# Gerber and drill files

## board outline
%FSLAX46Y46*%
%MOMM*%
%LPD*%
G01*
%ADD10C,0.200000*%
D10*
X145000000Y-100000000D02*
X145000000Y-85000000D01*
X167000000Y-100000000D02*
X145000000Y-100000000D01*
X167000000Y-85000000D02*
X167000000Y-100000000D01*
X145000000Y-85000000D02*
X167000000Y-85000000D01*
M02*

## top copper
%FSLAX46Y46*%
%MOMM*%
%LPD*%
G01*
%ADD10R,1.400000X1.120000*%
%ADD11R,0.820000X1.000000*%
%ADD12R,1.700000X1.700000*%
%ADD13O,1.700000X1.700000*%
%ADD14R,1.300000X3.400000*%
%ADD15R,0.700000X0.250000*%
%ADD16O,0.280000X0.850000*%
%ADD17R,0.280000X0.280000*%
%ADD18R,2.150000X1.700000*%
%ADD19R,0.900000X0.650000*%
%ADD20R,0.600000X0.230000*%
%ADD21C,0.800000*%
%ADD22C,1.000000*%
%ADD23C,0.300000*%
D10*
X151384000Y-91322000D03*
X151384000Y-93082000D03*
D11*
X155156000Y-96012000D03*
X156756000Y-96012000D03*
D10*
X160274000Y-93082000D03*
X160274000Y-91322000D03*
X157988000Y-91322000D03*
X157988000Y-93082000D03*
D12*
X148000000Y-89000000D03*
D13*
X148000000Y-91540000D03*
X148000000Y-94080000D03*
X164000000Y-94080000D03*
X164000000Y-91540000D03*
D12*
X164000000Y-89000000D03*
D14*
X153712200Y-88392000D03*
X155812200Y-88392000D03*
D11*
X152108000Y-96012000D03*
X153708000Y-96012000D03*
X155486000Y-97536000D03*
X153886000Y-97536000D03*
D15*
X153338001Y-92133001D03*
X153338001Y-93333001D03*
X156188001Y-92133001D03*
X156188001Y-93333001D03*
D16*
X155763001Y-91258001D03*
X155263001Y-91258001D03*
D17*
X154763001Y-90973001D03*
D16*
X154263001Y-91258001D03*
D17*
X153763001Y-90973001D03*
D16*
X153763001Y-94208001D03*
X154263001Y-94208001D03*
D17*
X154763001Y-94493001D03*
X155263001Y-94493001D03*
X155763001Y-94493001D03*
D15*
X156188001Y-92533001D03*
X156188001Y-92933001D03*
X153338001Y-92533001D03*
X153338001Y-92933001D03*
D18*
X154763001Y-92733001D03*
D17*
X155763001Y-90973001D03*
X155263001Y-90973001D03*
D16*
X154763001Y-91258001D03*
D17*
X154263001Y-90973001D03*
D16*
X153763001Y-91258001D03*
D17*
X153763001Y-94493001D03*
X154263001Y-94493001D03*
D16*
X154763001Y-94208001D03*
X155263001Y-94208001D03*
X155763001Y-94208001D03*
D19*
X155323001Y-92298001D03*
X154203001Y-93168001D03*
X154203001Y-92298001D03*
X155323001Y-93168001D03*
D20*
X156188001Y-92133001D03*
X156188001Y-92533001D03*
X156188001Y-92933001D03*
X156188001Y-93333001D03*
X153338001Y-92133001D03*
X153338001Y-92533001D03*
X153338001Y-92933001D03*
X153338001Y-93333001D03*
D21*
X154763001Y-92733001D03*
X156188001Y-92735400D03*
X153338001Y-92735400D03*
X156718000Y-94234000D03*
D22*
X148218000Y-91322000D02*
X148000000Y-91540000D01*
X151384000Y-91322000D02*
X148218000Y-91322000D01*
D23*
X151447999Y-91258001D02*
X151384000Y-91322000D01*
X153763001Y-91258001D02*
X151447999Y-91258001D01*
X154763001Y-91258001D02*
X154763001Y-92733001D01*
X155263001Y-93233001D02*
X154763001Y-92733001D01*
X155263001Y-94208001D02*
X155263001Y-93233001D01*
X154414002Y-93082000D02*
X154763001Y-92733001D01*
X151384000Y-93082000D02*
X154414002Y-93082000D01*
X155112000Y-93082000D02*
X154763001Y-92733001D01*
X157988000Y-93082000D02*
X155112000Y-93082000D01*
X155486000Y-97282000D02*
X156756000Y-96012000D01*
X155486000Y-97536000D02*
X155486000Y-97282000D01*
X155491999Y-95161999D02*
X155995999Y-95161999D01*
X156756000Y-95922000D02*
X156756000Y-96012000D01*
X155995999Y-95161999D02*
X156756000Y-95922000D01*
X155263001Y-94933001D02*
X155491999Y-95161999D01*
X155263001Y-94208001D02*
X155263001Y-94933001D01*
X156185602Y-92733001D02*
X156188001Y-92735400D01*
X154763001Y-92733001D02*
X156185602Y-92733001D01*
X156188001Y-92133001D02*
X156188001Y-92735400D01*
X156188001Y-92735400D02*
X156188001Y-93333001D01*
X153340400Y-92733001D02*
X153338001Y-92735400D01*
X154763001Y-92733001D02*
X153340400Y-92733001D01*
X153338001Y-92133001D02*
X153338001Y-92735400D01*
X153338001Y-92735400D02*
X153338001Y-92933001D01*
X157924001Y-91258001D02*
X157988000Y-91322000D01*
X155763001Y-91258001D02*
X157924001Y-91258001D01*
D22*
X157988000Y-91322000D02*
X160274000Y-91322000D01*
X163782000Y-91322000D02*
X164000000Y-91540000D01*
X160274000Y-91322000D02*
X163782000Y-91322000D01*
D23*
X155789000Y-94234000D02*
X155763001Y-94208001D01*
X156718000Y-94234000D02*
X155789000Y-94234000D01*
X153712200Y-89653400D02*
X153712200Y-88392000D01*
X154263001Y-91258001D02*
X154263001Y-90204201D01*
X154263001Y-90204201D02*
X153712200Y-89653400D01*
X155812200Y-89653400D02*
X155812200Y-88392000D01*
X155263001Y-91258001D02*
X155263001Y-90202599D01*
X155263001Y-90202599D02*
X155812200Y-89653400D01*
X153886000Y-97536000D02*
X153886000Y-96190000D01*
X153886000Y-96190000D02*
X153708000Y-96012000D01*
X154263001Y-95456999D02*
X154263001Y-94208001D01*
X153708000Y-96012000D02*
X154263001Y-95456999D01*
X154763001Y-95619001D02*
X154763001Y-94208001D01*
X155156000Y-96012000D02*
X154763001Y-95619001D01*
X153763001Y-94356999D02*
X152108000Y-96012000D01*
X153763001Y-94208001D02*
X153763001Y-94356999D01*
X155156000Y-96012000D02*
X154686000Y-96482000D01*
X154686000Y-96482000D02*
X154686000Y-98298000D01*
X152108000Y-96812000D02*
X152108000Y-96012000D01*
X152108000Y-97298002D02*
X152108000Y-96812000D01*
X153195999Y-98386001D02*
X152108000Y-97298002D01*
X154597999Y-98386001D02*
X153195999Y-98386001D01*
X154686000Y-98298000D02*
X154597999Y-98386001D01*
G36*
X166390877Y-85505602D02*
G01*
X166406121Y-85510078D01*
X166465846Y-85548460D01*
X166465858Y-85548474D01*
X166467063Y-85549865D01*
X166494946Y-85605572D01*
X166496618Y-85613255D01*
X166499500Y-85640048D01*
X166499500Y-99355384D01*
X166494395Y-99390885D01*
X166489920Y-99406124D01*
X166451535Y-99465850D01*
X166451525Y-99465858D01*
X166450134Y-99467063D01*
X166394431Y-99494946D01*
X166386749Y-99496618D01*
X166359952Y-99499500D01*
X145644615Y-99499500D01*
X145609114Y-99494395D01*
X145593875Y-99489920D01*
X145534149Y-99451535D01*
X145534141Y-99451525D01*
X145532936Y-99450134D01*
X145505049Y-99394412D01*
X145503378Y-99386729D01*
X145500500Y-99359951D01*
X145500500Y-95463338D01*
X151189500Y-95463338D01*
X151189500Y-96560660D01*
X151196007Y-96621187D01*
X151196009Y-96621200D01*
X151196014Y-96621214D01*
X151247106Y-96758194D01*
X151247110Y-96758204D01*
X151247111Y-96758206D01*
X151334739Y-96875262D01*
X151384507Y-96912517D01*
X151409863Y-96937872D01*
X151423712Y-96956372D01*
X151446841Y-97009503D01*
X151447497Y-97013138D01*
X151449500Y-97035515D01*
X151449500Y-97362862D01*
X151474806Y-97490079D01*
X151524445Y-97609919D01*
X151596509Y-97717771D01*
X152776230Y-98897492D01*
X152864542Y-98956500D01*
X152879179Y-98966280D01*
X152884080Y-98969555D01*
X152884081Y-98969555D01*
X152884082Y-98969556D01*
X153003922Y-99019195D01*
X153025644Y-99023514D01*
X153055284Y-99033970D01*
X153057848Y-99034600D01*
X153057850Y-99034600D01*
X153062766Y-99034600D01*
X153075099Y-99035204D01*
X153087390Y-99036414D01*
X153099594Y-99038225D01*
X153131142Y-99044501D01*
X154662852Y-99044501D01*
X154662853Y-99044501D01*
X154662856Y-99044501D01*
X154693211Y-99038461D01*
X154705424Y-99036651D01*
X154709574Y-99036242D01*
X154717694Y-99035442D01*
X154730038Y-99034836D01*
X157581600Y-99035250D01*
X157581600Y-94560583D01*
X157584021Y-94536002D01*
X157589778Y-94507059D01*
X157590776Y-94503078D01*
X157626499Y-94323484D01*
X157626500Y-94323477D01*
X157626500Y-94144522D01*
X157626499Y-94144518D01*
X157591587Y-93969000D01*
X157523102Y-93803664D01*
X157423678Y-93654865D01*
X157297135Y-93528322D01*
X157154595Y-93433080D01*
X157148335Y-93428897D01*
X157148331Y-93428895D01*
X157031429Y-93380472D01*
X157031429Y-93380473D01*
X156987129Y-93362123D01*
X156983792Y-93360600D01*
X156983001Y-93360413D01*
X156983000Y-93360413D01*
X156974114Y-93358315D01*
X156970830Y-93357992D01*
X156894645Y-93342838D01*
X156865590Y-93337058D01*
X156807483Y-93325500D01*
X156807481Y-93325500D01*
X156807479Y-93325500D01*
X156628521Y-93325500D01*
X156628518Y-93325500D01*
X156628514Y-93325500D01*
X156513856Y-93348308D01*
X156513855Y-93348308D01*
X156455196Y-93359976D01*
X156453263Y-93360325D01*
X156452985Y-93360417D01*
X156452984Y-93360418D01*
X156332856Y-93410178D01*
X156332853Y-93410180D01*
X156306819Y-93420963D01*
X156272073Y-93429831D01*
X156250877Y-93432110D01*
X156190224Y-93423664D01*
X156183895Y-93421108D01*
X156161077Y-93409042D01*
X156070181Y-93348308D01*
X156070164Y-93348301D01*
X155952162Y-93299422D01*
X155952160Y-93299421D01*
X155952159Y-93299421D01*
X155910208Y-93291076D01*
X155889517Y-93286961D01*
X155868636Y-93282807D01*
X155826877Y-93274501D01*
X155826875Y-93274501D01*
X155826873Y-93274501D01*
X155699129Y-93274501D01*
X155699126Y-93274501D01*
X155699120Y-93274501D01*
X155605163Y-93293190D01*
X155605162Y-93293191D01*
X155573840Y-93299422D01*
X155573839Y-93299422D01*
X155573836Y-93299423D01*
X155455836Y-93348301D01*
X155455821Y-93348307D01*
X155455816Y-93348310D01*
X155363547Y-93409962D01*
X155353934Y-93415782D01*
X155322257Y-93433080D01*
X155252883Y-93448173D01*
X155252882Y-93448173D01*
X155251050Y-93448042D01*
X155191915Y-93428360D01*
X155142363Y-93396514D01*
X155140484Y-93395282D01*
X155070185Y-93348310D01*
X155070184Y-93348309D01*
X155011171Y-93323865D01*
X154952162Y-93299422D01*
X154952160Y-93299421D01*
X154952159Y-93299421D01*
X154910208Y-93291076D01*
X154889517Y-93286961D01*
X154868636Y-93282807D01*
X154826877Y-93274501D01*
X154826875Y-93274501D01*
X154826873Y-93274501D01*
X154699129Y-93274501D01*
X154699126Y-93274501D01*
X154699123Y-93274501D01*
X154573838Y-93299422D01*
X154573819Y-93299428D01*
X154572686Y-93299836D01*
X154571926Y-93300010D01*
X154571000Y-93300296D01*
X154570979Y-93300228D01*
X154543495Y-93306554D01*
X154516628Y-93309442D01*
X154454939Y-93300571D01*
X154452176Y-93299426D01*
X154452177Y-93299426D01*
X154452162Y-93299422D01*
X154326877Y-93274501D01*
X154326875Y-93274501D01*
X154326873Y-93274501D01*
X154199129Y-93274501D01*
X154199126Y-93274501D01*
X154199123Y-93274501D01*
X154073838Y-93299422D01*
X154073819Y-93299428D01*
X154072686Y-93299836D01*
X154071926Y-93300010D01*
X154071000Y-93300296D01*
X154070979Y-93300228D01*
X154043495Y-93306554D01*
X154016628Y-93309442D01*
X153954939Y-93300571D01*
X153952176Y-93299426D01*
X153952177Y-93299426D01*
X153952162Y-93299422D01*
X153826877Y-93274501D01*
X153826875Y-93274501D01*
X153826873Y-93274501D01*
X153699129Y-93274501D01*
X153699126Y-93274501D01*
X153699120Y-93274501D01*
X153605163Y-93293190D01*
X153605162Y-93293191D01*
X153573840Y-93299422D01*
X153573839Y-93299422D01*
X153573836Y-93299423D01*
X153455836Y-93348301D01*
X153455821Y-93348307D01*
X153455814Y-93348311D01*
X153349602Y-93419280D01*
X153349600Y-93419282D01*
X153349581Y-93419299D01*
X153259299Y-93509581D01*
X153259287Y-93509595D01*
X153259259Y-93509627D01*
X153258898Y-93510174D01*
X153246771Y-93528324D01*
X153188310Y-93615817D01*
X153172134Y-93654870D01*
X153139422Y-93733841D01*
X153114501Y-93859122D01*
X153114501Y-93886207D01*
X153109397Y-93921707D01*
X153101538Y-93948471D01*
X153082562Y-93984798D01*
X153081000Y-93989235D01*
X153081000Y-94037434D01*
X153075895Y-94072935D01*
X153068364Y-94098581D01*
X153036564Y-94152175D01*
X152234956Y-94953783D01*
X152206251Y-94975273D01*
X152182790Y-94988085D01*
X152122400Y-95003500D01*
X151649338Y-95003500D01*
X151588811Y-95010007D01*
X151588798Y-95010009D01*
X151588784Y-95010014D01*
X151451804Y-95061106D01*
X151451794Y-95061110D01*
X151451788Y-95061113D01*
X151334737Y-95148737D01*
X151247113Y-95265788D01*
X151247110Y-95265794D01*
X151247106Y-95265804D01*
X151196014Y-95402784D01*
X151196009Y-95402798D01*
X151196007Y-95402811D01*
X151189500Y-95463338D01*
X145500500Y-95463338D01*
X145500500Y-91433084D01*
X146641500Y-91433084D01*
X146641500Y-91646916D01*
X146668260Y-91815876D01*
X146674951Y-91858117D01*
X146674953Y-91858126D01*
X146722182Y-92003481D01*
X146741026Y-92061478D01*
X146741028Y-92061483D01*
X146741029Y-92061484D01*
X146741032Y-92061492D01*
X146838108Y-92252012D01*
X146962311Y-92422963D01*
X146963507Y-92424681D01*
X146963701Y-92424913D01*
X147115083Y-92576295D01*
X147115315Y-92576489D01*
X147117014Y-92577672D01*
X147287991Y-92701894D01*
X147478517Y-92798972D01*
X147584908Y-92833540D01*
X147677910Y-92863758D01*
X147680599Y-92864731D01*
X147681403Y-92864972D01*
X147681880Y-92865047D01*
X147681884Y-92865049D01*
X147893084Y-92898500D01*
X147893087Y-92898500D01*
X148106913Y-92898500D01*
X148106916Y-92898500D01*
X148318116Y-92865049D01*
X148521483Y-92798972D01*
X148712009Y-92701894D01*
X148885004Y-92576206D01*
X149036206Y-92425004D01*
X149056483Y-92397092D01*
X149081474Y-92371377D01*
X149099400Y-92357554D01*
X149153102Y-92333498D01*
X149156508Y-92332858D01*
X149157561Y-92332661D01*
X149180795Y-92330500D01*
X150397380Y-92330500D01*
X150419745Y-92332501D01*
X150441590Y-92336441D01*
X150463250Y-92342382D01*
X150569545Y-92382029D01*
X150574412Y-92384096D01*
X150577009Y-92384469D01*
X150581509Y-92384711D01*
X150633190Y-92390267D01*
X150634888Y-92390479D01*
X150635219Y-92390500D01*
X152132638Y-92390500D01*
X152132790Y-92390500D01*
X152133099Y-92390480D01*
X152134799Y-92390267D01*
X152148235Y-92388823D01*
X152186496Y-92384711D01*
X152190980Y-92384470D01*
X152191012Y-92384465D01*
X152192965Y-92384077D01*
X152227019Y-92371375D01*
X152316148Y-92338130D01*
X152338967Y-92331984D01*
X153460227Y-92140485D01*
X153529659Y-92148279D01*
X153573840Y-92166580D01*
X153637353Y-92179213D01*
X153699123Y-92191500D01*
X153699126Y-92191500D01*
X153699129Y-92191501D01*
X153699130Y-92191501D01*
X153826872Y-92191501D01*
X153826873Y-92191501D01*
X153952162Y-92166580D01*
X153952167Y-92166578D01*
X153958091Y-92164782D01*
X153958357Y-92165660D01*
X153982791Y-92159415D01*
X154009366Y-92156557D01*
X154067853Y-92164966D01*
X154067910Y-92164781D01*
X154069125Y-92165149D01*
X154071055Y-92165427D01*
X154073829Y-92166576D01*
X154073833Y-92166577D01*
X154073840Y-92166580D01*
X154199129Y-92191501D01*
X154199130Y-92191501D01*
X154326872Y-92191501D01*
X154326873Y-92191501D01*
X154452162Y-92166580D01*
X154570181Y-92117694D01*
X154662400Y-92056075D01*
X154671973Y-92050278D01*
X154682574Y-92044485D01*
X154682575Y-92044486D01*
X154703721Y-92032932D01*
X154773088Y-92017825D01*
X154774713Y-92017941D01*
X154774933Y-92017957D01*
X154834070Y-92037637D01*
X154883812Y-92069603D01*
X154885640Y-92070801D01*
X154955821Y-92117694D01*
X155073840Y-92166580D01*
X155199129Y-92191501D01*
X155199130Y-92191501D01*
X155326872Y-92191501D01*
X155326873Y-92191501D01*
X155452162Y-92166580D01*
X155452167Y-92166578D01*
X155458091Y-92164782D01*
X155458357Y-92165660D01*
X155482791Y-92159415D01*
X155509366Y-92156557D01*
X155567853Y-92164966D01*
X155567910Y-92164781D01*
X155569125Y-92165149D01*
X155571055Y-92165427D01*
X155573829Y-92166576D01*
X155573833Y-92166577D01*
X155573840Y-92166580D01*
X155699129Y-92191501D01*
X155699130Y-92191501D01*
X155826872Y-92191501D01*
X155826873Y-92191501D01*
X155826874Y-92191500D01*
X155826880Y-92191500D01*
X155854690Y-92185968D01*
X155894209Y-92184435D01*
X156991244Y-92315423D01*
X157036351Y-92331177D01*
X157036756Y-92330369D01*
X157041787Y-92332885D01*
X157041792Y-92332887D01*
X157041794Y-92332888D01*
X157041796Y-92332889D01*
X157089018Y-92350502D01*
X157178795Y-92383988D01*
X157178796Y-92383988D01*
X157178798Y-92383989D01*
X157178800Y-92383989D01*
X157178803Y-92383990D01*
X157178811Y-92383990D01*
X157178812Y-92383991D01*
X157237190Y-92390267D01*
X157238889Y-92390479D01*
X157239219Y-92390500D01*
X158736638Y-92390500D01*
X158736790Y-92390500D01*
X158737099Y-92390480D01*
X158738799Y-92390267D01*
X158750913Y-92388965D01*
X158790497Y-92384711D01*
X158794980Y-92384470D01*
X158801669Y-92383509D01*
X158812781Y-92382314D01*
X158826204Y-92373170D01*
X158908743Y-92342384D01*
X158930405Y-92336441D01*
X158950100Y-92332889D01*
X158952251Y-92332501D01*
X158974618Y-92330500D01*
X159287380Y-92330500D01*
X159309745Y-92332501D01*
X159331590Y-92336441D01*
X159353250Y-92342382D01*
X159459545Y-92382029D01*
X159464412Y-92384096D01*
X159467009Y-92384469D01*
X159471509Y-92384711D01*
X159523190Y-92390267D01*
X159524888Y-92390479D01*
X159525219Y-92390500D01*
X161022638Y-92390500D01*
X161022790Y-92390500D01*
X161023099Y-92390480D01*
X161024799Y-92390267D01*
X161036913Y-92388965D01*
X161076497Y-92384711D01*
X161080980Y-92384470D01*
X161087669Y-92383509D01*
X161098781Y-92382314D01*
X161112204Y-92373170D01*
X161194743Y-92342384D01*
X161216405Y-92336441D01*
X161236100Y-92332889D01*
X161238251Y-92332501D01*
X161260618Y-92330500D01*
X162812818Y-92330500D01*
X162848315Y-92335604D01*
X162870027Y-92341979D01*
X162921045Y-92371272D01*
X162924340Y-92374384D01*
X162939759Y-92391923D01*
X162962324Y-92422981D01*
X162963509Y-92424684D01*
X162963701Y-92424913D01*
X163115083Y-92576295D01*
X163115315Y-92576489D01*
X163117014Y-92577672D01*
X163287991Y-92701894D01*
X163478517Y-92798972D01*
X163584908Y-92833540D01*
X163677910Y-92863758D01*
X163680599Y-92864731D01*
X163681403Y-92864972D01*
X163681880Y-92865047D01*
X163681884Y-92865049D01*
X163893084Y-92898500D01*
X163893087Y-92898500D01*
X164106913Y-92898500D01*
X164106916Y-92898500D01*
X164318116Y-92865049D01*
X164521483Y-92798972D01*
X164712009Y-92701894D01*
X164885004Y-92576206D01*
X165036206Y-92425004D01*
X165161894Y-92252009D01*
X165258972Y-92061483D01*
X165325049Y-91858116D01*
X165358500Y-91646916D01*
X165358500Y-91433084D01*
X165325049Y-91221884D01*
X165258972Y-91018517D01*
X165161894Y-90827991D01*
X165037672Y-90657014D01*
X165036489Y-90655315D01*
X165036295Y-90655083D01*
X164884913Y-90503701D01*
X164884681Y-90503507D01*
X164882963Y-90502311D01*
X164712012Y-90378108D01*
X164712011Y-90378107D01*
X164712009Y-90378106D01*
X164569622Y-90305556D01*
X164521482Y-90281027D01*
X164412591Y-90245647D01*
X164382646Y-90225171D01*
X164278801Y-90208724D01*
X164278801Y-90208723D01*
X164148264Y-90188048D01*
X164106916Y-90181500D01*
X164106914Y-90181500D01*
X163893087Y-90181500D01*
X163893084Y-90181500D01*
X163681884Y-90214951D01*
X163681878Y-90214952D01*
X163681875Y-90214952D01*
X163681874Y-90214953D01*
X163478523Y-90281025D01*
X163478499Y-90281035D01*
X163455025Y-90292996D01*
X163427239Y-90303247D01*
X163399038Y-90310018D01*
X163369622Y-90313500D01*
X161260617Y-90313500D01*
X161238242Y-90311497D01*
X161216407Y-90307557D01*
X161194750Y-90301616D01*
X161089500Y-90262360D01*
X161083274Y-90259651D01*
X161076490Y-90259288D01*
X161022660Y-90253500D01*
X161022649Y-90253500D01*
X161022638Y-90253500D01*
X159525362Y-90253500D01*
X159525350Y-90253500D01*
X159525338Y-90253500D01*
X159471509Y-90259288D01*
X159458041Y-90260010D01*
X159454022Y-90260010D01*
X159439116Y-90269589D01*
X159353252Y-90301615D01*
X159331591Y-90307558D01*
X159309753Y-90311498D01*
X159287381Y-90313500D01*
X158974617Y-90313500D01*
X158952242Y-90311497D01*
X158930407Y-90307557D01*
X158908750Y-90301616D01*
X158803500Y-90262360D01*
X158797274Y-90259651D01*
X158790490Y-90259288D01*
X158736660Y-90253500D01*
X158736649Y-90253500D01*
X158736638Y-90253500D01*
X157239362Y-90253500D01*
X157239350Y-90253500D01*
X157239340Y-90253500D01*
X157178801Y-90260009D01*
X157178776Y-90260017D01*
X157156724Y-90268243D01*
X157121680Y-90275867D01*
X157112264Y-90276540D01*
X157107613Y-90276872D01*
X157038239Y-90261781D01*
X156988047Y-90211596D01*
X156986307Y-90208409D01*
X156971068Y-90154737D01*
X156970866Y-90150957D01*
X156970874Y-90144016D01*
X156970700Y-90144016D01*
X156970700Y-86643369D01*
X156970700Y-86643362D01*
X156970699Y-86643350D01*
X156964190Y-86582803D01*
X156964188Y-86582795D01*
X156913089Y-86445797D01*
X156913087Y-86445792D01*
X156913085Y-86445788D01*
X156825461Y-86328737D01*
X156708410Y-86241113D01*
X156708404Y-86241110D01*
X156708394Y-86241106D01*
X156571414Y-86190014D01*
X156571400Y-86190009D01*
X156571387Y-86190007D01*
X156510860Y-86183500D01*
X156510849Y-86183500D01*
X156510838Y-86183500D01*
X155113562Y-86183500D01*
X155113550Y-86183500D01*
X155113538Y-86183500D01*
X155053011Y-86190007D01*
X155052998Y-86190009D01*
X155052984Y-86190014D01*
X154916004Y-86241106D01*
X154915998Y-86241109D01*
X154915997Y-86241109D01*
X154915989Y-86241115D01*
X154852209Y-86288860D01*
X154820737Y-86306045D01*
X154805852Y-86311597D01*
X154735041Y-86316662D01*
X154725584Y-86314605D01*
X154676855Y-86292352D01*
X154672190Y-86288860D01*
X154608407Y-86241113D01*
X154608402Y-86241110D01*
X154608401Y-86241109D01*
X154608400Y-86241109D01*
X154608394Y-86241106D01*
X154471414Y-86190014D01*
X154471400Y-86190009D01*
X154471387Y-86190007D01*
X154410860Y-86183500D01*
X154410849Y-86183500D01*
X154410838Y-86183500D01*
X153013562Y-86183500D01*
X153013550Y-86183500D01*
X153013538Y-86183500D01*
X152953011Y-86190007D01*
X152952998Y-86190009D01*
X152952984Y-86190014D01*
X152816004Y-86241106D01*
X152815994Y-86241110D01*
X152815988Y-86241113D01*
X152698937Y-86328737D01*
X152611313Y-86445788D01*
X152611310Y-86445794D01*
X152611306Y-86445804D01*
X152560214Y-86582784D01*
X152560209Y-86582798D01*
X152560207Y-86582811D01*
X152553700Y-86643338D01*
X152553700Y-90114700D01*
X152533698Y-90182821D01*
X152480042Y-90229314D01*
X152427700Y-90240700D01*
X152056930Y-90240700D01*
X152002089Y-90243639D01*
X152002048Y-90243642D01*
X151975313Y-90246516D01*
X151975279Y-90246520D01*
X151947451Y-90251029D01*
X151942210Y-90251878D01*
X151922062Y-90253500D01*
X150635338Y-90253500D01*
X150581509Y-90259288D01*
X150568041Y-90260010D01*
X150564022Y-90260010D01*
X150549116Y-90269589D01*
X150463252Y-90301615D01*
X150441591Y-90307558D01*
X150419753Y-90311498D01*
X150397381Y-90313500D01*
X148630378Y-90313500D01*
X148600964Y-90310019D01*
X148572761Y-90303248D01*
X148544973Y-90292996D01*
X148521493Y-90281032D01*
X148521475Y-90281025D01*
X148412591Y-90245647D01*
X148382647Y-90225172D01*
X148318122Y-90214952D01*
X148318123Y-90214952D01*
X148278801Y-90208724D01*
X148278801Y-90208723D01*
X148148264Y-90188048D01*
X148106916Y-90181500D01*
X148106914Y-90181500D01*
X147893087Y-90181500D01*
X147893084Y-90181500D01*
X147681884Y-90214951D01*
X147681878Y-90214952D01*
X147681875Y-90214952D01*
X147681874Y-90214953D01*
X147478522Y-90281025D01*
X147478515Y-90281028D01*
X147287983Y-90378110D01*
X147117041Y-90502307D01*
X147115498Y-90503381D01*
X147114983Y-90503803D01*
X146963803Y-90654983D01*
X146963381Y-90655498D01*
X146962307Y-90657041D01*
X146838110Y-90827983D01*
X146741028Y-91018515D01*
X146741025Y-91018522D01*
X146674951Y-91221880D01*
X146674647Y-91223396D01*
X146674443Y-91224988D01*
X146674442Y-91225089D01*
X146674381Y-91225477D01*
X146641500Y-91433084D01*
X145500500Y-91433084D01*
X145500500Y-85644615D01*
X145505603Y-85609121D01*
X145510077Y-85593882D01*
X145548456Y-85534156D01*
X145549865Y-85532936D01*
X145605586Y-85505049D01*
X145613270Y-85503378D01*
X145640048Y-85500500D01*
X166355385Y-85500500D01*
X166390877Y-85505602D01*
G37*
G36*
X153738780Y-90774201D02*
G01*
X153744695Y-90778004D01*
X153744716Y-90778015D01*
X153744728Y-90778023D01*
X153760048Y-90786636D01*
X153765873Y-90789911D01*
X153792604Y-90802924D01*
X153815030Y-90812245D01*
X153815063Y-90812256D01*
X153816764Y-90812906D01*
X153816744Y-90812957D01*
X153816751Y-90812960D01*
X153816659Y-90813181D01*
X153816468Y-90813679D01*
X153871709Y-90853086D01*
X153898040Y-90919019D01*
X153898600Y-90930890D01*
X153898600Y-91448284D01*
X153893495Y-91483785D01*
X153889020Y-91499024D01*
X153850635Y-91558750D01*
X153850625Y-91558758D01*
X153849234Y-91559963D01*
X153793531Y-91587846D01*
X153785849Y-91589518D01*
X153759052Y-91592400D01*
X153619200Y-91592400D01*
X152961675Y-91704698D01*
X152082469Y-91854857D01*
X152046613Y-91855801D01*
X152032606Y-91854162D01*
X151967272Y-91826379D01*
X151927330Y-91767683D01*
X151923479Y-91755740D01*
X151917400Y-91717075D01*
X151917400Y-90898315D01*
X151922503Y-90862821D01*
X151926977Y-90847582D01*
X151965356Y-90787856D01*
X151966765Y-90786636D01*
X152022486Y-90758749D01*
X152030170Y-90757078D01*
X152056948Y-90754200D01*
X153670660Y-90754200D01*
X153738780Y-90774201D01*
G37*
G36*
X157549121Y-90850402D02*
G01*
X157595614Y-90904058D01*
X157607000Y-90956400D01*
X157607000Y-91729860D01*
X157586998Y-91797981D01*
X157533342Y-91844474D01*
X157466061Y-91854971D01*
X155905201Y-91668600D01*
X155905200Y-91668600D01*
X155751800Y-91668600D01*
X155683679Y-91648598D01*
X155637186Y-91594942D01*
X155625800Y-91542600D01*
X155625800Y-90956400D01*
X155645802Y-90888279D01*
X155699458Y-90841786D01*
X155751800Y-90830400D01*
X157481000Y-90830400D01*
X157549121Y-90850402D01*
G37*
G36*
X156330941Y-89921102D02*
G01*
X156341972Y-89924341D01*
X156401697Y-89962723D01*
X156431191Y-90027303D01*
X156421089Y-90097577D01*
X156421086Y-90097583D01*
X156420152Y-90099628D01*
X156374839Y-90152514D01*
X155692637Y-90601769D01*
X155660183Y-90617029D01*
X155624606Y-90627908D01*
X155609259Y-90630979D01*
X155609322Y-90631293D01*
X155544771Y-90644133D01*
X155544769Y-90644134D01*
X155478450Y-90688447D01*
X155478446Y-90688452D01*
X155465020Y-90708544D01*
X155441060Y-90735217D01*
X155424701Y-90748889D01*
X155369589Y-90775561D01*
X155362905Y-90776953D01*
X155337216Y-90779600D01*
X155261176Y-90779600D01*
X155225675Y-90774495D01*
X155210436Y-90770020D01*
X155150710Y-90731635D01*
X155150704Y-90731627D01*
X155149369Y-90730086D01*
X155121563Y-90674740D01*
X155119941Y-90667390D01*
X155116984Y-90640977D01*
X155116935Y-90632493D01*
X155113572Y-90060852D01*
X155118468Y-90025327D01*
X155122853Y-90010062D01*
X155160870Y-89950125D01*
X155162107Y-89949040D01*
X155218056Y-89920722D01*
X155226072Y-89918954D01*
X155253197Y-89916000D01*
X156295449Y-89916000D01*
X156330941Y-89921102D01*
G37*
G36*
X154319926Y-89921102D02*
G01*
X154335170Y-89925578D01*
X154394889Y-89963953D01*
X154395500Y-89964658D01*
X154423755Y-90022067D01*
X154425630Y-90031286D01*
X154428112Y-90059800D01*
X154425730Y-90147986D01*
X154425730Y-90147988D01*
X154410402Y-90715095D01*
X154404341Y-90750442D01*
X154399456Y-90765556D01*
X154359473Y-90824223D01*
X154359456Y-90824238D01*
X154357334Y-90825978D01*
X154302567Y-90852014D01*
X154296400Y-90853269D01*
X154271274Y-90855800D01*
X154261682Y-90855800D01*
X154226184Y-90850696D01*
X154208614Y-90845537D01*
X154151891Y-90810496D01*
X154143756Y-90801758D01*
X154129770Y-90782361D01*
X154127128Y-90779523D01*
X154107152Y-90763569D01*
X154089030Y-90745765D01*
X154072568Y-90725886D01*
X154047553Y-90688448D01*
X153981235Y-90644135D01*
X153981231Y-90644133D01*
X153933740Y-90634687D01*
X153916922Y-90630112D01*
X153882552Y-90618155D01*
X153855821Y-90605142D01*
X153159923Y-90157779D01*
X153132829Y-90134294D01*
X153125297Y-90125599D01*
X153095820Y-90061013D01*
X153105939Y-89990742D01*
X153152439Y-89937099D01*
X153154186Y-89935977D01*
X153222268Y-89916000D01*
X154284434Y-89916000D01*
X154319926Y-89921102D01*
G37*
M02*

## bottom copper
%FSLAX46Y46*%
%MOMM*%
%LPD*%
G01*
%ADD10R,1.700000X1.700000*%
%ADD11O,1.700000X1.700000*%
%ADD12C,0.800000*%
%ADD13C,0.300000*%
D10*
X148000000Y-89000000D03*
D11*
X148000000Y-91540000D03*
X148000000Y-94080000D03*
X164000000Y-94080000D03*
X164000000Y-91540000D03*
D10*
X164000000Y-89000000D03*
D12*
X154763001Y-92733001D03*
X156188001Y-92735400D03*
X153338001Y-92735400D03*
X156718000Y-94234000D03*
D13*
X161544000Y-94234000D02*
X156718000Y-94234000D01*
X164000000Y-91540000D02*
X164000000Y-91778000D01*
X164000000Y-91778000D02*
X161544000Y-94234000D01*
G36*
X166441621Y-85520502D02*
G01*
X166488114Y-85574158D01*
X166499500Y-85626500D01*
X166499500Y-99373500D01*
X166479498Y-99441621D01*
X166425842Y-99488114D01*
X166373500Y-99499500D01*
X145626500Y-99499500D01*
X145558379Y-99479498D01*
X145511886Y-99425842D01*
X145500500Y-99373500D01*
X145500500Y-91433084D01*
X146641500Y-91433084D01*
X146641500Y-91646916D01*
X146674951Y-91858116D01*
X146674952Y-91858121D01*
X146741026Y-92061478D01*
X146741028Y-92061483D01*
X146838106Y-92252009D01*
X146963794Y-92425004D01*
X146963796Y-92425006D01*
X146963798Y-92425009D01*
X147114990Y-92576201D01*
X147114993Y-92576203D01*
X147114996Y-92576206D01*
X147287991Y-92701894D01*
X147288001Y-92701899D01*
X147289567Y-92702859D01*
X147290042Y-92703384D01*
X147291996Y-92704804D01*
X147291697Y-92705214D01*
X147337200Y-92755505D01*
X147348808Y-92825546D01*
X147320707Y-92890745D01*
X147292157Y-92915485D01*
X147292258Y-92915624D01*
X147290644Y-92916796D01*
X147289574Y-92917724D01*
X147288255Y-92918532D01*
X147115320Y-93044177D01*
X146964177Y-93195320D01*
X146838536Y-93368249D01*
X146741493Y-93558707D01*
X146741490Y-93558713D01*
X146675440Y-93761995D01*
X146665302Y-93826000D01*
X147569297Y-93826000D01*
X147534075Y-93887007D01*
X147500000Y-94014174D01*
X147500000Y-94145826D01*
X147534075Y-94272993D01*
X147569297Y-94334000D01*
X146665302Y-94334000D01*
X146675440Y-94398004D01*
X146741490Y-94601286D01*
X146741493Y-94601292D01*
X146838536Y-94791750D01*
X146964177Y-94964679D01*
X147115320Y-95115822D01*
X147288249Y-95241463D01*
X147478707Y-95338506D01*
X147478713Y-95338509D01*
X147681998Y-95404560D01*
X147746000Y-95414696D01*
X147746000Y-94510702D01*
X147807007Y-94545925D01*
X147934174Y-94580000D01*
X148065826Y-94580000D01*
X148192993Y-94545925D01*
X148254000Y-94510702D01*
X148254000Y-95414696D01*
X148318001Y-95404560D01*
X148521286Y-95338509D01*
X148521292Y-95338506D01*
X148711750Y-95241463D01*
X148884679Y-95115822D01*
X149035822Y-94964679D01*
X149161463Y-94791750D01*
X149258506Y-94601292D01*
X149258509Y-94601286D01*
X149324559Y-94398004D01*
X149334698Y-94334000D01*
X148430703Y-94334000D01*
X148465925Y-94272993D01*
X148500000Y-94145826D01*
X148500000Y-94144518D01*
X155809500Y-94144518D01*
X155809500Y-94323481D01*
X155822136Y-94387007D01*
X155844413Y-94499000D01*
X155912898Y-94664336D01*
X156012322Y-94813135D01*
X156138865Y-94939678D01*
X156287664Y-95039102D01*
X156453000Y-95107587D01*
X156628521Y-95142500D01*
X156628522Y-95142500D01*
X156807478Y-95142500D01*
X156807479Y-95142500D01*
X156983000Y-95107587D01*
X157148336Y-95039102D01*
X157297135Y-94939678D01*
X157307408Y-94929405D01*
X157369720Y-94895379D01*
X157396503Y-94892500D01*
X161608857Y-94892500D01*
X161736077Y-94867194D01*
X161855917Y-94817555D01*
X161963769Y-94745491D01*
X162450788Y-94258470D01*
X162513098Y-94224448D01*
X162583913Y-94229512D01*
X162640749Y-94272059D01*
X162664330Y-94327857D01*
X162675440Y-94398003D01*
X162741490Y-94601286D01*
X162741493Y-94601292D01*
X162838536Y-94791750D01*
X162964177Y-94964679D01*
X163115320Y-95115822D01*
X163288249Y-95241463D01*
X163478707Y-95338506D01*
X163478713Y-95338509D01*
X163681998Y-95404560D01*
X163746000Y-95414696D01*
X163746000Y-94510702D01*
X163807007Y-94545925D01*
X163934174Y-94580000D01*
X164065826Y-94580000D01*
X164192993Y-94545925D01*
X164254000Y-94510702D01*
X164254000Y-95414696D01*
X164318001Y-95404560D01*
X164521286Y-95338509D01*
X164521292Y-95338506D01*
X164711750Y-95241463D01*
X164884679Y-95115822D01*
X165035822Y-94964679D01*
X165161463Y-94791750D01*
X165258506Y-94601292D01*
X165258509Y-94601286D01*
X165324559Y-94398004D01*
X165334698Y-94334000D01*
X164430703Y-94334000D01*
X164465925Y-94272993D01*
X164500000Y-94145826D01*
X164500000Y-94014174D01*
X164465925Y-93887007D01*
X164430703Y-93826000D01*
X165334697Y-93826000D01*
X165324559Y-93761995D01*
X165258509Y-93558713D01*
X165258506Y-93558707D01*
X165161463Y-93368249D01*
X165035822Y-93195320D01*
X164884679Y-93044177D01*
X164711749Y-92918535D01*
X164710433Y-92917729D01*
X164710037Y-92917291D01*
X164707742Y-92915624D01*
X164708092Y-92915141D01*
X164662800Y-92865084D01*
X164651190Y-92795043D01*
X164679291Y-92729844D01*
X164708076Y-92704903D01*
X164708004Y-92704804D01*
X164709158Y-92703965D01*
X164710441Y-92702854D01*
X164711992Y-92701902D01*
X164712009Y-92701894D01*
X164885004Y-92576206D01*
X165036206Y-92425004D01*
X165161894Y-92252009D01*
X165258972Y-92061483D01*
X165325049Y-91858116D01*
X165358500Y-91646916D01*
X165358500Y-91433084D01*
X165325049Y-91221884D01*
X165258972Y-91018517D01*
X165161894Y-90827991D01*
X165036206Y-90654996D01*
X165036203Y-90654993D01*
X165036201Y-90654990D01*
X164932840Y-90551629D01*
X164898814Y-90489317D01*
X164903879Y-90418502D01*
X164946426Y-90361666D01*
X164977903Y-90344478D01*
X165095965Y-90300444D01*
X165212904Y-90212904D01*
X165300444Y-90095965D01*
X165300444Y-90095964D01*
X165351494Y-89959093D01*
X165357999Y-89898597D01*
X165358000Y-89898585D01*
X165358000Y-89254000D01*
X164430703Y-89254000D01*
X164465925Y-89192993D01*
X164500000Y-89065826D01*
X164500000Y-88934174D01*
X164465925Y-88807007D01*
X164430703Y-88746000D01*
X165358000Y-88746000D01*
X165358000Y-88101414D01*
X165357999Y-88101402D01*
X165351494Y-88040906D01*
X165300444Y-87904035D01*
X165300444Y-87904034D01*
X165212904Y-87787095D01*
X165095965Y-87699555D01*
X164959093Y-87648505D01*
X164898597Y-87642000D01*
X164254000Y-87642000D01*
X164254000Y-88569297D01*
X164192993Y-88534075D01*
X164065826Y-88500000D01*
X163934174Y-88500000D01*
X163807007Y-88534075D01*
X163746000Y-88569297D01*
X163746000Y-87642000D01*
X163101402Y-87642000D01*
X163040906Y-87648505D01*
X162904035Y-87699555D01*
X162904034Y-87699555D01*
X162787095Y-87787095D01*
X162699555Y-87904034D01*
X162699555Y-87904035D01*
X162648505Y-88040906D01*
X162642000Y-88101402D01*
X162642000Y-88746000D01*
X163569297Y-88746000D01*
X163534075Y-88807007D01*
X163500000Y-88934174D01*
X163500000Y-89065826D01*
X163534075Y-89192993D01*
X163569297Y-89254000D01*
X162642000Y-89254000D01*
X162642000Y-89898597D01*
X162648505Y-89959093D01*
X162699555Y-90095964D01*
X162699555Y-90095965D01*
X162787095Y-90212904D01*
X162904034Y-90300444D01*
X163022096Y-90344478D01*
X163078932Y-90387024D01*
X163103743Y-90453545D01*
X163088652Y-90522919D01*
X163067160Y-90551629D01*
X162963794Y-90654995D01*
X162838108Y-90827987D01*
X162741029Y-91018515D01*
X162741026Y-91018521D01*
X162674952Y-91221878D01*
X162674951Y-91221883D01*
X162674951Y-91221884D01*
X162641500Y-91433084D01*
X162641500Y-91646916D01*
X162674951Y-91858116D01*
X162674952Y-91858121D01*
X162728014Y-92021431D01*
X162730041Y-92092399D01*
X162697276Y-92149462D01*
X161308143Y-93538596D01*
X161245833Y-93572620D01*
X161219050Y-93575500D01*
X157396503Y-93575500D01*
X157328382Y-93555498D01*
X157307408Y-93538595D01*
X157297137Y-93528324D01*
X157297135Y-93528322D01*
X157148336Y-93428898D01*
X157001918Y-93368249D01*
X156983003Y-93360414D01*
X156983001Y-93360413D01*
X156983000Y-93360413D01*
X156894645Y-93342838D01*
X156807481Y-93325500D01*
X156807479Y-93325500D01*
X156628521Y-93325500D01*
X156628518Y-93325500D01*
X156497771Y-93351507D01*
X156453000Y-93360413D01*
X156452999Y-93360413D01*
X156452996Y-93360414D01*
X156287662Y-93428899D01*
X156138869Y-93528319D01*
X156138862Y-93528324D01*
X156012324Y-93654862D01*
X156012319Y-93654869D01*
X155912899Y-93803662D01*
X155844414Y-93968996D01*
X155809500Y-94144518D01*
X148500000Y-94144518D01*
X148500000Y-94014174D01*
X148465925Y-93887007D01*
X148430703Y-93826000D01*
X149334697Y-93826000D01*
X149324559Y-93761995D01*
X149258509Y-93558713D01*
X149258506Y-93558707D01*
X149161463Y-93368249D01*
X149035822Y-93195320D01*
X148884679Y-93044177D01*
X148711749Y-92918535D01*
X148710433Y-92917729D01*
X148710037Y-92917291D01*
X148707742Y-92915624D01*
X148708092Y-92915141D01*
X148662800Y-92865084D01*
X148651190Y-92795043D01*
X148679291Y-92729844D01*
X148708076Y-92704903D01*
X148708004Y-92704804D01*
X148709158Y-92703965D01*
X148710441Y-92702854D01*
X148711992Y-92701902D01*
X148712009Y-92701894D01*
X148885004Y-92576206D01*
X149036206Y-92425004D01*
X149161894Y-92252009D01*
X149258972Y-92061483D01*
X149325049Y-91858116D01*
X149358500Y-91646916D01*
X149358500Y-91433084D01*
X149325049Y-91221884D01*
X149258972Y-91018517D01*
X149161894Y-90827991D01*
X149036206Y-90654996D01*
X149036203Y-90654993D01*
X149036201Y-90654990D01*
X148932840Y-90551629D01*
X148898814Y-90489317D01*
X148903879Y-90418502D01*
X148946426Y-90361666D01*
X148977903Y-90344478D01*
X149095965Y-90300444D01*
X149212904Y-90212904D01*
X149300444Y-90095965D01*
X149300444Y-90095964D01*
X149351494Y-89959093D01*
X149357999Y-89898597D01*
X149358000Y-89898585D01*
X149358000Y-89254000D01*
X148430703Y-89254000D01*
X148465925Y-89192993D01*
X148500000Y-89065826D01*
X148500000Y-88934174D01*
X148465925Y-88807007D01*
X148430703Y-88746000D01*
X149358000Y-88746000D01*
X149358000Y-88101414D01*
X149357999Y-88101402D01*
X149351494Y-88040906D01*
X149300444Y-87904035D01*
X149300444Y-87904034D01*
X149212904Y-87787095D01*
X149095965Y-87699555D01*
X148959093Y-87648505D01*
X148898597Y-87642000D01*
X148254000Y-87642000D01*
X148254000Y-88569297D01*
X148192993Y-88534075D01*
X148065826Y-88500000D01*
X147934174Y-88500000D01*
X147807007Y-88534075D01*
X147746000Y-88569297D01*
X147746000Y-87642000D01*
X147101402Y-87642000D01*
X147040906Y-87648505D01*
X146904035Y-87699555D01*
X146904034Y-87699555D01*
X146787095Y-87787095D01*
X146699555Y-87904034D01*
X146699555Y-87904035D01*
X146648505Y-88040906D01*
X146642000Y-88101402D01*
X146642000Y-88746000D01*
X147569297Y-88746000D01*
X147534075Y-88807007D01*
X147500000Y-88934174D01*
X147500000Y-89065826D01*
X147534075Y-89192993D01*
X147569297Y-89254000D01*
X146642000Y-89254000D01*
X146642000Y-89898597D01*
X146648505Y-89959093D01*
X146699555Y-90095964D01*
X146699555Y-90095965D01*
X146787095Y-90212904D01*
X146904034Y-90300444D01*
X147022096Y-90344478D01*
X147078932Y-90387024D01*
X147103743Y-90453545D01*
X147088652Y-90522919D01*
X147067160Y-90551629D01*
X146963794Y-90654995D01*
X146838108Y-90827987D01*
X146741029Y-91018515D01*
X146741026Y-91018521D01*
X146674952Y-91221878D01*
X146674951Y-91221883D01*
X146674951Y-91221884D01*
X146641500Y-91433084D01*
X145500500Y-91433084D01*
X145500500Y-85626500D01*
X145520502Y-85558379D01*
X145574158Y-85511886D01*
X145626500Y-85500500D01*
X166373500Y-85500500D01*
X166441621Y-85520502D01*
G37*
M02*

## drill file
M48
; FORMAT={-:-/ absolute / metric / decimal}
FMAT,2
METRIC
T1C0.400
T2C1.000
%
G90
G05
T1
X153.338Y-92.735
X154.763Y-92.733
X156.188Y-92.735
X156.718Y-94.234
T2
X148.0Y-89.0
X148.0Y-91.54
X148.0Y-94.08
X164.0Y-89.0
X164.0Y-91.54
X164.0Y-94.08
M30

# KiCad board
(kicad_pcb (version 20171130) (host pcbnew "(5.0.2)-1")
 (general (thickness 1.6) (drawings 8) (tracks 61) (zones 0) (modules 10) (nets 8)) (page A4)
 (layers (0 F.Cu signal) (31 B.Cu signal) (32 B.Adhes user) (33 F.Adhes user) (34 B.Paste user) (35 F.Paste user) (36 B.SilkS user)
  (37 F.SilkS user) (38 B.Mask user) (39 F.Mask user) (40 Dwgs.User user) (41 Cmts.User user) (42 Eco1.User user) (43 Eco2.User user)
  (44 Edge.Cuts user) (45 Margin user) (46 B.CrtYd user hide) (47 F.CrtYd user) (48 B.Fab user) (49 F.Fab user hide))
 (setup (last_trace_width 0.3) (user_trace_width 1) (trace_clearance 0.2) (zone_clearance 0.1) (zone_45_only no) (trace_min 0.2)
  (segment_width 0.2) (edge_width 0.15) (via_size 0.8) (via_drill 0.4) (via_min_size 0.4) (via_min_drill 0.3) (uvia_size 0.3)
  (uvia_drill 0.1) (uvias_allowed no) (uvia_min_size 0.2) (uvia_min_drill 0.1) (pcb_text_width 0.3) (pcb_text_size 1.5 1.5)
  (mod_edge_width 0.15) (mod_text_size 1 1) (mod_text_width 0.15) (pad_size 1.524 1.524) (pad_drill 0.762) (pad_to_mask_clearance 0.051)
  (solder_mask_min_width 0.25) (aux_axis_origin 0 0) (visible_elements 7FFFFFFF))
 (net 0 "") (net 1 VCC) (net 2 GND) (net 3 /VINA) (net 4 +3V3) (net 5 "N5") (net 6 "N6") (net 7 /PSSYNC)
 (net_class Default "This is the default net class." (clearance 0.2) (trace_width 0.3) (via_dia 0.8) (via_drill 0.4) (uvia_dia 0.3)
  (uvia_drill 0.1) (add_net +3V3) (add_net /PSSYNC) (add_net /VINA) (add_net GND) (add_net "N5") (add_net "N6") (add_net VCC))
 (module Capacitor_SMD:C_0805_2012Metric (layer F.Cu) (at 151.384 92.202 270)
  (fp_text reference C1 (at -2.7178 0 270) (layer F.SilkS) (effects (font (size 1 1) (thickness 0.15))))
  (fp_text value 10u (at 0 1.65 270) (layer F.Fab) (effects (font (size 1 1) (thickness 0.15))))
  (pad 1 smd rect (at -0.88 0 270) (size 1.12 1.4) (layers F.Cu F.Paste F.Mask) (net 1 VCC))
  (pad 2 smd rect (at 0.88 0 270) (size 1.12 1.4) (layers F.Cu F.Paste F.Mask) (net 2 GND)))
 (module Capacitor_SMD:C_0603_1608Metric (layer F.Cu) (at 155.956 96.012)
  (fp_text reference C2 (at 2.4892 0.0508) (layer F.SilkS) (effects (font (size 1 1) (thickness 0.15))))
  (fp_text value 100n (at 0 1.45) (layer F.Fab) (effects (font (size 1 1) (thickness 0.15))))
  (pad 1 smd rect (at -0.8 0) (size 0.82 1) (layers F.Cu F.Paste F.Mask) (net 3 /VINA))
  (pad 2 smd rect (at 0.8 0) (size 0.82 1) (layers F.Cu F.Paste F.Mask) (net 2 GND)))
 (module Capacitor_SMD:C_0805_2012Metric (layer F.Cu) (at 160.274 92.202 270)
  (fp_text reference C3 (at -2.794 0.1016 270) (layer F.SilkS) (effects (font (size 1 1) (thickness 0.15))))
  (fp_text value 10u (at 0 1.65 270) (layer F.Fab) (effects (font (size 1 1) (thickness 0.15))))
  (pad 2 smd rect (at 0.88 0 270) (size 1.12 1.4) (layers F.Cu F.Paste F.Mask) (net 2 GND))
  (pad 1 smd rect (at -0.88 0 270) (size 1.12 1.4) (layers F.Cu F.Paste F.Mask) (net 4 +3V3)))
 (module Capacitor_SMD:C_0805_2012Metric (layer F.Cu) (at 157.988 92.202 270)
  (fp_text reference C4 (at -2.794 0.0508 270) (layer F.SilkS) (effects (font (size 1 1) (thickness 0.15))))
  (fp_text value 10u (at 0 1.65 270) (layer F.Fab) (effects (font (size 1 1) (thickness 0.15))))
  (pad 1 smd rect (at -0.88 0 270) (size 1.12 1.4) (layers F.Cu F.Paste F.Mask) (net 4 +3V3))
  (pad 2 smd rect (at 0.88 0 270) (size 1.12 1.4) (layers F.Cu F.Paste F.Mask) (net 2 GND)))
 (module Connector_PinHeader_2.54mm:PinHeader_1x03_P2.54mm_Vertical (layer F.Cu) (at 148 89)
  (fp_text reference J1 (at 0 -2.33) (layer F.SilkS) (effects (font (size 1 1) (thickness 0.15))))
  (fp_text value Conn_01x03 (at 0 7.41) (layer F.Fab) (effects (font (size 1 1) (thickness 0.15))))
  (pad 1 thru_hole rect (at 0 0) (size 1.7 1.7) (drill 1) (layers *.Cu *.Mask) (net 2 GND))
  (pad 2 thru_hole oval (at 0 2.54) (size 1.7 1.7) (drill 1) (layers *.Cu *.Mask) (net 1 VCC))
  (pad 3 thru_hole oval (at 0 5.08) (size 1.7 1.7) (drill 1) (layers *.Cu *.Mask) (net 2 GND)))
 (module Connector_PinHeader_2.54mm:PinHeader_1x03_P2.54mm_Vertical (layer F.Cu) (at 164 89)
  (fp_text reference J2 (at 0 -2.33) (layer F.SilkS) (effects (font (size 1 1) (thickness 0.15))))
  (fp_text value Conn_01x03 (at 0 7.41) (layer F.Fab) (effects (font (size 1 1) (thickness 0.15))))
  (pad 3 thru_hole oval (at 0 5.08) (size 1.7 1.7) (drill 1) (layers *.Cu *.Mask) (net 2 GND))
  (pad 2 thru_hole oval (at 0 2.54) (size 1.7 1.7) (drill 1) (layers *.Cu *.Mask) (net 4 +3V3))
  (pad 1 thru_hole rect (at 0 0) (size 1.7 1.7) (drill 1) (layers *.Cu *.Mask) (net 2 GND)))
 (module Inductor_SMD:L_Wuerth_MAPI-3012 (layer F.Cu) (at 154.7622 88.392)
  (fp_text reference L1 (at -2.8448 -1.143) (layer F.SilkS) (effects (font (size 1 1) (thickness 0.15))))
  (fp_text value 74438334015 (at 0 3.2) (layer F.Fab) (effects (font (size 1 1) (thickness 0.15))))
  (pad 1 smd rect (at -1.05 0) (size 1.3 3.4) (layers F.Cu F.Paste F.Mask) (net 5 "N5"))
  (pad 2 smd rect (at 1.05 0) (size 1.3 3.4) (layers F.Cu F.Paste F.Mask) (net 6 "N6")))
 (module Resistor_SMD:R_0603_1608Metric (layer F.Cu) (at 152.908 96.012)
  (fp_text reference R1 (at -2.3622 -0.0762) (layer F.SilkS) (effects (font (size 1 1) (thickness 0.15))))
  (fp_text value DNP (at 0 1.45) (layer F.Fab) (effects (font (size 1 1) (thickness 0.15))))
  (pad 1 smd rect (at -0.8 0) (size 0.82 1) (layers F.Cu F.Paste F.Mask) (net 3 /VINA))
  (pad 2 smd rect (at 0.8 0) (size 0.82 1) (layers F.Cu F.Paste F.Mask) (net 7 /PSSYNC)))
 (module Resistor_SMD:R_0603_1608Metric (layer F.Cu) (at 154.686 97.536)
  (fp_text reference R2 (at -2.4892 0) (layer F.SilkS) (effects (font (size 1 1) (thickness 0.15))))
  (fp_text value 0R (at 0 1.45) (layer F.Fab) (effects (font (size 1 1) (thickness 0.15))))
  (pad 2 smd rect (at 0.8 0) (size 0.82 1) (layers F.Cu F.Paste F.Mask) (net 2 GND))
  (pad 1 smd rect (at -0.8 0) (size 0.82 1) (layers F.Cu F.Paste F.Mask) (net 7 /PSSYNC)))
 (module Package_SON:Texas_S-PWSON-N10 (layer F.Cu) (at 154.763001 92.733001 270)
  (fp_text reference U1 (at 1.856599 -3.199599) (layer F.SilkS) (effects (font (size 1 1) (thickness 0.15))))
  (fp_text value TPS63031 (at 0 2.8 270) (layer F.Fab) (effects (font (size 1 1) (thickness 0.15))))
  (pad 11 smd rect (at -0.6 1.425 270) (size 0.25 0.7) (layers F.Cu F.Mask) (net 2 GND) (solder_paste_margin -0.05))
  (pad 11 smd rect (at 0.6 1.425 270) (size 0.25 0.7) (layers F.Cu F.Mask) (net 2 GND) (solder_paste_margin -0.05))
  (pad 11 smd rect (at -0.6 -1.425 270) (size 0.25 0.7) (layers F.Cu F.Mask) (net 2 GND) (solder_paste_margin -0.05))
  (pad 11 smd rect (at 0.6 -1.425 270) (size 0.25 0.7) (layers F.Cu F.Mask) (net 2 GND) (solder_paste_margin -0.05))
  (pad 1 smd oval (at -1.475 -1 270) (size 0.85 0.28) (layers F.Cu F.Paste F.Mask) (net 4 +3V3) (solder_mask_margin 0.07)
   (solder_paste_margin -0.025))
  (pad 2 smd oval (at -1.475 -0.5 270) (size 0.85 0.28) (layers F.Cu F.Paste F.Mask) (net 6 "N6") (solder_mask_margin 0.07)
   (solder_paste_margin -0.025))
  (pad 3 smd rect (at -1.76 0 270) (size 0.28 0.28) (layers F.Cu F.Paste F.Mask) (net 2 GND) (solder_mask_margin 0.07)
   (solder_paste_margin -0.025))
  (pad 4 smd oval (at -1.475 0.5 270) (size 0.85 0.28) (layers F.Cu F.Paste F.Mask) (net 5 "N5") (solder_mask_margin 0.07)
   (solder_paste_margin -0.025))
  (pad 5 smd rect (at -1.76 1 270) (size 0.28 0.28) (layers F.Cu F.Paste F.Mask) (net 1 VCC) (solder_mask_margin 0.07)
   (solder_paste_margin -0.025))
  (pad 6 smd oval (at 1.475 1 270) (size 0.85 0.28) (layers F.Cu F.Paste F.Mask) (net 3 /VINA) (solder_mask_margin 0.07)
   (solder_paste_margin -0.025))
  (pad 7 smd oval (at 1.475 0.5 270) (size 0.85 0.28) (layers F.Cu F.Paste F.Mask) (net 7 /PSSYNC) (solder_mask_margin 0.07)
   (solder_paste_margin -0.025))
  (pad 8 smd rect (at 1.76 0 270) (size 0.28 0.28) (layers F.Cu F.Paste F.Mask) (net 3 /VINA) (solder_mask_margin 0.07)
   (solder_paste_margin -0.025))
  (pad 9 smd rect (at 1.76 -0.5 270) (size 0.28 0.28) (layers F.Cu F.Paste F.Mask) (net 2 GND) (solder_mask_margin 0.07)
   (solder_paste_margin -0.025))
  (pad 10 smd rect (at 1.76 -1 270) (size 0.28 0.28) (layers F.Cu F.Paste F.Mask) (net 4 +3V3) (solder_mask_margin 0.07)
   (solder_paste_margin -0.025))
  (pad 11 smd rect (at -0.2 -1.425 270) (size 0.25 0.7) (layers F.Cu F.Mask) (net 2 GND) (solder_paste_margin -0.05))
  (pad 11 smd rect (at 0.2 -1.425 270) (size 0.25 0.7) (layers F.Cu F.Mask) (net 2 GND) (solder_paste_margin -0.05))
  (pad 11 smd rect (at -0.2 1.425 270) (size 0.25 0.7) (layers F.Cu F.Mask) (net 2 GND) (solder_paste_margin -0.05))
  (pad 11 smd rect (at 0.2 1.425 270) (size 0.25 0.7) (layers F.Cu F.Mask) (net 2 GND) (solder_paste_margin -0.05))
  (pad 11 smd rect (at 0 0 270) (size 1.7 2.15) (layers F.Cu F.Mask) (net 2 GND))
  (pad 1 smd rect (at -1.76 -1 270) (size 0.28 0.28) (layers F.Cu F.Paste F.Mask) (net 4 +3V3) (solder_mask_margin 0.07)
   (solder_paste_margin -0.025))
  (pad 2 smd rect (at -1.76 -0.5 270) (size 0.28 0.28) (layers F.Cu F.Paste F.Mask) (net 6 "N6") (solder_mask_margin 0.07)
   (solder_paste_margin -0.025))
  (pad 3 smd oval (at -1.475 0 270) (size 0.85 0.28) (layers F.Cu F.Paste F.Mask) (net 2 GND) (solder_mask_margin 0.07)
   (solder_paste_margin -0.025))
  (pad 4 smd rect (at -1.76 0.5 270) (size 0.28 0.28) (layers F.Cu F.Paste F.Mask) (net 5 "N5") (solder_mask_margin 0.07)
   (solder_paste_margin -0.025))
  (pad 5 smd oval (at -1.475 1 270) (size 0.85 0.28) (layers F.Cu F.Paste F.Mask) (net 1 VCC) (solder_mask_margin 0.07)
   (solder_paste_margin -0.025))
  (pad 6 smd rect (at 1.76 1 270) (size 0.28 0.28) (layers F.Cu F.Paste F.Mask) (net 3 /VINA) (solder_mask_margin 0.07)
   (solder_paste_margin -0.025))
  (pad 7 smd rect (at 1.76 0.5 270) (size 0.28 0.28) (layers F.Cu F.Paste F.Mask) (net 7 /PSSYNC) (solder_mask_margin 0.07)
   (solder_paste_margin -0.025))
  (pad 8 smd oval (at 1.475 0 270) (size 0.85 0.28) (layers F.Cu F.Paste F.Mask) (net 3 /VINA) (solder_mask_margin 0.07)
   (solder_paste_margin -0.025))
  (pad 9 smd oval (at 1.475 -0.5 270) (size 0.85 0.28) (layers F.Cu F.Paste F.Mask) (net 2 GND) (solder_mask_margin 0.07)
   (solder_paste_margin -0.025))
  (pad 10 smd oval (at 1.475 -1 270) (size 0.85 0.28) (layers F.Cu F.Paste F.Mask) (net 4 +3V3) (solder_mask_margin 0.07)
   (solder_paste_margin -0.025))
  (pad 11 smd rect (at -0.435 -0.56 270) (size 0.65 0.9) (layers F.Cu F.Paste F.Mask) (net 2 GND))
  (pad 11 smd rect (at 0.435 0.56 270) (size 0.65 0.9) (layers F.Cu F.Paste F.Mask) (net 2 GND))
  (pad 11 smd rect (at -0.435 0.56 270) (size 0.65 0.9) (layers F.Cu F.Paste F.Mask) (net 2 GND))
  (pad 11 smd rect (at 0.435 -0.56 270) (size 0.65 0.9) (layers F.Cu F.Paste F.Mask) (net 2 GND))
  (pad 11 smd rect (at -0.6 -1.425 270) (size 0.23 0.6) (layers F.Cu F.Paste F.Mask) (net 2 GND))
  (pad 11 smd rect (at -0.2 -1.425 270) (size 0.23 0.6) (layers F.Cu F.Paste F.Mask) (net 2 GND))
  (pad 11 smd rect (at 0.2 -1.425 270) (size 0.23 0.6) (layers F.Cu F.Paste F.Mask) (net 2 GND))
  (pad 11 smd rect (at 0.6 -1.425 270) (size 0.23 0.6) (layers F.Cu F.Paste F.Mask) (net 2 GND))
  (pad 11 smd rect (at -0.6 1.425 270) (size 0.23 0.6) (layers F.Cu F.Paste F.Mask) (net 2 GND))
  (pad 11 smd rect (at -0.2 1.425 270) (size 0.23 0.6) (layers F.Cu F.Paste F.Mask) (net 2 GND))
  (pad 11 smd rect (at 0.2 1.425 270) (size 0.23 0.6) (layers F.Cu F.Paste F.Mask) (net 2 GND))
  (pad 11 smd rect (at 0.6 1.425 270) (size 0.23 0.6) (layers F.Cu F.Paste F.Mask) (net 2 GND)))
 (gr_line (start 145 100) (end 145 85) (layer Edge.Cuts) (width 0.2))
 (gr_line (start 167 100) (end 145 100) (layer Edge.Cuts) (width 0.2))
 (gr_line (start 167 85) (end 167 100) (layer Edge.Cuts) (width 0.2))
 (gr_line (start 145 85) (end 167 85) (layer Edge.Cuts) (width 0.2))
 (segment (start 148.218 91.322) (end 148 91.54) (width 1) (layer F.Cu) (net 1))
 (segment (start 151.384 91.322) (end 148.218 91.322) (width 1) (layer F.Cu) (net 1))
 (segment (start 151.447999 91.258001) (end 151.384 91.322) (width 0.3) (layer F.Cu) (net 1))
 (segment (start 153.763001 91.258001) (end 151.447999 91.258001) (width 0.3) (layer F.Cu) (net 1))
 (segment (start 154.763001 91.258001) (end 154.763001 92.733001) (width 0.3) (layer F.Cu) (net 2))
 (segment (start 155.263001 93.233001) (end 154.763001 92.733001) (width 0.3) (layer F.Cu) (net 2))
 (segment (start 155.263001 94.208001) (end 155.263001 93.233001) (width 0.3) (layer F.Cu) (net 2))
 (segment (start 154.414002 93.082) (end 154.763001 92.733001) (width 0.3) (layer F.Cu) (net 2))
 (segment (start 151.384 93.082) (end 154.414002 93.082) (width 0.3) (layer F.Cu) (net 2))
 (segment (start 155.112 93.082) (end 154.763001 92.733001) (width 0.3) (layer F.Cu) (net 2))
 (segment (start 157.988 93.082) (end 155.112 93.082) (width 0.3) (layer F.Cu) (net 2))
 (segment (start 155.486 97.282) (end 156.756 96.012) (width 0.3) (layer F.Cu) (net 2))
 (segment (start 155.486 97.536) (end 155.486 97.282) (width 0.3) (layer F.Cu) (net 2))
 (segment (start 155.491999 95.161999) (end 155.995999 95.161999) (width 0.3) (layer F.Cu) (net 2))
 (segment (start 156.756 95.922) (end 156.756 96.012) (width 0.3) (layer F.Cu) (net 2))
 (segment (start 155.995999 95.161999) (end 156.756 95.922) (width 0.3) (layer F.Cu) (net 2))
 (segment (start 155.263001 94.933001) (end 155.491999 95.161999) (width 0.3) (layer F.Cu) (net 2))
 (segment (start 155.263001 94.208001) (end 155.263001 94.933001) (width 0.3) (layer F.Cu) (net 2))
 (via (at 154.763001 92.733001) (size 0.8) (drill 0.4) (layers F.Cu B.Cu) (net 2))
 (via (at 156.188001 92.7354) (size 0.8) (drill 0.4) (layers F.Cu B.Cu) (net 2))
 (segment (start 156.185602 92.733001) (end 156.188001 92.7354) (width 0.3) (layer F.Cu) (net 2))
 (segment (start 154.763001 92.733001) (end 156.185602 92.733001) (width 0.3) (layer F.Cu) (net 2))
 (segment (start 156.188001 92.133001) (end 156.188001 92.7354) (width 0.3) (layer F.Cu) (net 2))
 (segment (start 156.188001 92.7354) (end 156.188001 93.333001) (width 0.3) (layer F.Cu) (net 2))
 (via (at 153.338001 92.7354) (size 0.8) (drill 0.4) (layers F.Cu B.Cu) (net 2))
 (segment (start 153.3404 92.733001) (end 153.338001 92.7354) (width 0.3) (layer F.Cu) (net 2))
 (segment (start 154.763001 92.733001) (end 153.3404 92.733001) (width 0.3) (layer F.Cu) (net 2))
 (segment (start 153.338001 92.133001) (end 153.338001 92.7354) (width 0.3) (layer F.Cu) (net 2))
 (segment (start 153.338001 92.7354) (end 153.338001 92.933001) (width 0.3) (layer F.Cu) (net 2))
 (segment (start 157.924001 91.258001) (end 157.988 91.322) (width 0.3) (layer F.Cu) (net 4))
 (segment (start 155.763001 91.258001) (end 157.924001 91.258001) (width 0.3) (layer F.Cu) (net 4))
 (segment (start 157.988 91.322) (end 160.274 91.322) (width 1) (layer F.Cu) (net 4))
 (segment (start 163.782 91.322) (end 164 91.54) (width 1) (layer F.Cu) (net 4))
 (segment (start 160.274 91.322) (end 163.782 91.322) (width 1) (layer F.Cu) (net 4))
 (via (at 156.718 94.234) (size 0.8) (drill 0.4) (layers F.Cu B.Cu) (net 4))
 (segment (start 155.789 94.234) (end 155.763001 94.208001) (width 0.3) (layer F.Cu) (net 4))
 (segment (start 156.718 94.234) (end 155.789 94.234) (width 0.3) (layer F.Cu) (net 4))
 (segment (start 161.544 94.234) (end 156.718 94.234) (width 0.3) (layer B.Cu) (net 4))
 (segment (start 164 91.54) (end 164 91.778) (width 0.3) (layer B.Cu) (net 4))
 (segment (start 164 91.778) (end 161.544 94.234) (width 0.3) (layer B.Cu) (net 4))
 (segment (start 153.7122 89.6534) (end 153.7122 88.392) (width 0.3) (layer F.Cu) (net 5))
 (segment (start 154.263001 91.258001) (end 154.263001 90.204201) (width 0.3) (layer F.Cu) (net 5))
 (segment (start 154.263001 90.204201) (end 153.7122 89.6534) (width 0.3) (layer F.Cu) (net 5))
 (segment (start 155.8122 89.6534) (end 155.8122 88.392) (width 0.3) (layer F.Cu) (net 6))
 (segment (start 155.263001 91.258001) (end 155.263001 90.202599) (width 0.3) (layer F.Cu) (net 6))
 (segment (start 155.263001 90.202599) (end 155.8122 89.6534) (width 0.3) (layer F.Cu) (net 6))
 (segment (start 153.886 97.536) (end 153.886 96.19) (width 0.3) (layer F.Cu) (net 7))
 (segment (start 153.886 96.19) (end 153.708 96.012) (width 0.3) (layer F.Cu) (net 7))
 (segment (start 154.263001 95.456999) (end 154.263001 94.208001) (width 0.3) (layer F.Cu) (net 7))
 (segment (start 153.708 96.012) (end 154.263001 95.456999) (width 0.3) (layer F.Cu) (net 7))
 (segment (start 154.763001 95.619001) (end 154.763001 94.208001) (width 0.3) (layer F.Cu) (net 3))
 (segment (start 155.156 96.012) (end 154.763001 95.619001) (width 0.3) (layer F.Cu) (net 3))
 (segment (start 153.763001 94.356999) (end 152.108 96.012) (width 0.3) (layer F.Cu) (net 3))
 (segment (start 153.763001 94.208001) (end 153.763001 94.356999) (width 0.3) (layer F.Cu) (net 3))
 (segment (start 155.156 96.012) (end 154.686 96.482) (width 0.3) (layer F.Cu) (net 3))
 (segment (start 154.686 96.482) (end 154.686 98.298) (width 0.3) (layer F.Cu) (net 3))
 (segment (start 152.108 96.812) (end 152.108 96.012) (width 0.3) (layer F.Cu) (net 3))
 (segment (start 152.108 97.298002) (end 152.108 96.812) (width 0.3) (layer F.Cu) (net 3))
 (segment (start 153.195999 98.386001) (end 152.108 97.298002) (width 0.3) (layer F.Cu) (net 3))
 (segment (start 154.597999 98.386001) (end 153.195999 98.386001) (width 0.3) (layer F.Cu) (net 3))
 (segment (start 154.686 98.298) (end 154.597999 98.386001) (width 0.3) (layer F.Cu) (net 3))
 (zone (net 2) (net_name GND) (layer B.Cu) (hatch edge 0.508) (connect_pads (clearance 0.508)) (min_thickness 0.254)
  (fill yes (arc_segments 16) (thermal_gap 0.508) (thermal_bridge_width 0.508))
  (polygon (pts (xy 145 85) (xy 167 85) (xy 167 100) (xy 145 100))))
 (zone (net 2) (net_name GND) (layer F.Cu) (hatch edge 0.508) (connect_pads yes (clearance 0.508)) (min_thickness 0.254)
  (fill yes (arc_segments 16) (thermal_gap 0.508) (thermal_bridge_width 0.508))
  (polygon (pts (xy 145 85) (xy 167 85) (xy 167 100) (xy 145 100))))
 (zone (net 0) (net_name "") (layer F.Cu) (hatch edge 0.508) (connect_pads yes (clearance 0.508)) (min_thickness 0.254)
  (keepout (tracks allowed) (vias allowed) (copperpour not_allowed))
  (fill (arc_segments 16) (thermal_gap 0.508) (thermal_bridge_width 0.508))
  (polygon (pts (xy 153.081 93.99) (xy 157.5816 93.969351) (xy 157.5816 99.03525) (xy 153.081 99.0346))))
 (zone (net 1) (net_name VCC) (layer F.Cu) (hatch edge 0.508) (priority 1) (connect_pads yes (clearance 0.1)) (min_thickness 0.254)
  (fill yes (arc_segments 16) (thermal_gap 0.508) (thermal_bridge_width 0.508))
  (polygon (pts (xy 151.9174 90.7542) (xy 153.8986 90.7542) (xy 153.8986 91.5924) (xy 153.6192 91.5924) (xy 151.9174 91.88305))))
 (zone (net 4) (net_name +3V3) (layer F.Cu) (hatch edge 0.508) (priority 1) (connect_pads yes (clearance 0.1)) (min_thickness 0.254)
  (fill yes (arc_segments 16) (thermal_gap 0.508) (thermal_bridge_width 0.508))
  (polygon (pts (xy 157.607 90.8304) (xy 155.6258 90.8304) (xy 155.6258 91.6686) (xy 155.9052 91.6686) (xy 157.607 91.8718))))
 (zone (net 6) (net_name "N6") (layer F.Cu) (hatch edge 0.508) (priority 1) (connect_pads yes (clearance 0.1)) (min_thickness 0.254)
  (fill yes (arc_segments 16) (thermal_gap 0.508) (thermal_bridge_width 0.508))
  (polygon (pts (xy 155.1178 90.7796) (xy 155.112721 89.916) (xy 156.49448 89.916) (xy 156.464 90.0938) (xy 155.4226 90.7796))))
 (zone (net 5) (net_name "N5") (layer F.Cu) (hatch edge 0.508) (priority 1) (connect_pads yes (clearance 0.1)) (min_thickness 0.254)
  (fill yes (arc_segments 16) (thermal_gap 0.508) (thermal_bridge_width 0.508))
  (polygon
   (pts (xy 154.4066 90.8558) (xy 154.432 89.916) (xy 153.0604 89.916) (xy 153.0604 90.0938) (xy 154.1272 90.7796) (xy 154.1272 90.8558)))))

